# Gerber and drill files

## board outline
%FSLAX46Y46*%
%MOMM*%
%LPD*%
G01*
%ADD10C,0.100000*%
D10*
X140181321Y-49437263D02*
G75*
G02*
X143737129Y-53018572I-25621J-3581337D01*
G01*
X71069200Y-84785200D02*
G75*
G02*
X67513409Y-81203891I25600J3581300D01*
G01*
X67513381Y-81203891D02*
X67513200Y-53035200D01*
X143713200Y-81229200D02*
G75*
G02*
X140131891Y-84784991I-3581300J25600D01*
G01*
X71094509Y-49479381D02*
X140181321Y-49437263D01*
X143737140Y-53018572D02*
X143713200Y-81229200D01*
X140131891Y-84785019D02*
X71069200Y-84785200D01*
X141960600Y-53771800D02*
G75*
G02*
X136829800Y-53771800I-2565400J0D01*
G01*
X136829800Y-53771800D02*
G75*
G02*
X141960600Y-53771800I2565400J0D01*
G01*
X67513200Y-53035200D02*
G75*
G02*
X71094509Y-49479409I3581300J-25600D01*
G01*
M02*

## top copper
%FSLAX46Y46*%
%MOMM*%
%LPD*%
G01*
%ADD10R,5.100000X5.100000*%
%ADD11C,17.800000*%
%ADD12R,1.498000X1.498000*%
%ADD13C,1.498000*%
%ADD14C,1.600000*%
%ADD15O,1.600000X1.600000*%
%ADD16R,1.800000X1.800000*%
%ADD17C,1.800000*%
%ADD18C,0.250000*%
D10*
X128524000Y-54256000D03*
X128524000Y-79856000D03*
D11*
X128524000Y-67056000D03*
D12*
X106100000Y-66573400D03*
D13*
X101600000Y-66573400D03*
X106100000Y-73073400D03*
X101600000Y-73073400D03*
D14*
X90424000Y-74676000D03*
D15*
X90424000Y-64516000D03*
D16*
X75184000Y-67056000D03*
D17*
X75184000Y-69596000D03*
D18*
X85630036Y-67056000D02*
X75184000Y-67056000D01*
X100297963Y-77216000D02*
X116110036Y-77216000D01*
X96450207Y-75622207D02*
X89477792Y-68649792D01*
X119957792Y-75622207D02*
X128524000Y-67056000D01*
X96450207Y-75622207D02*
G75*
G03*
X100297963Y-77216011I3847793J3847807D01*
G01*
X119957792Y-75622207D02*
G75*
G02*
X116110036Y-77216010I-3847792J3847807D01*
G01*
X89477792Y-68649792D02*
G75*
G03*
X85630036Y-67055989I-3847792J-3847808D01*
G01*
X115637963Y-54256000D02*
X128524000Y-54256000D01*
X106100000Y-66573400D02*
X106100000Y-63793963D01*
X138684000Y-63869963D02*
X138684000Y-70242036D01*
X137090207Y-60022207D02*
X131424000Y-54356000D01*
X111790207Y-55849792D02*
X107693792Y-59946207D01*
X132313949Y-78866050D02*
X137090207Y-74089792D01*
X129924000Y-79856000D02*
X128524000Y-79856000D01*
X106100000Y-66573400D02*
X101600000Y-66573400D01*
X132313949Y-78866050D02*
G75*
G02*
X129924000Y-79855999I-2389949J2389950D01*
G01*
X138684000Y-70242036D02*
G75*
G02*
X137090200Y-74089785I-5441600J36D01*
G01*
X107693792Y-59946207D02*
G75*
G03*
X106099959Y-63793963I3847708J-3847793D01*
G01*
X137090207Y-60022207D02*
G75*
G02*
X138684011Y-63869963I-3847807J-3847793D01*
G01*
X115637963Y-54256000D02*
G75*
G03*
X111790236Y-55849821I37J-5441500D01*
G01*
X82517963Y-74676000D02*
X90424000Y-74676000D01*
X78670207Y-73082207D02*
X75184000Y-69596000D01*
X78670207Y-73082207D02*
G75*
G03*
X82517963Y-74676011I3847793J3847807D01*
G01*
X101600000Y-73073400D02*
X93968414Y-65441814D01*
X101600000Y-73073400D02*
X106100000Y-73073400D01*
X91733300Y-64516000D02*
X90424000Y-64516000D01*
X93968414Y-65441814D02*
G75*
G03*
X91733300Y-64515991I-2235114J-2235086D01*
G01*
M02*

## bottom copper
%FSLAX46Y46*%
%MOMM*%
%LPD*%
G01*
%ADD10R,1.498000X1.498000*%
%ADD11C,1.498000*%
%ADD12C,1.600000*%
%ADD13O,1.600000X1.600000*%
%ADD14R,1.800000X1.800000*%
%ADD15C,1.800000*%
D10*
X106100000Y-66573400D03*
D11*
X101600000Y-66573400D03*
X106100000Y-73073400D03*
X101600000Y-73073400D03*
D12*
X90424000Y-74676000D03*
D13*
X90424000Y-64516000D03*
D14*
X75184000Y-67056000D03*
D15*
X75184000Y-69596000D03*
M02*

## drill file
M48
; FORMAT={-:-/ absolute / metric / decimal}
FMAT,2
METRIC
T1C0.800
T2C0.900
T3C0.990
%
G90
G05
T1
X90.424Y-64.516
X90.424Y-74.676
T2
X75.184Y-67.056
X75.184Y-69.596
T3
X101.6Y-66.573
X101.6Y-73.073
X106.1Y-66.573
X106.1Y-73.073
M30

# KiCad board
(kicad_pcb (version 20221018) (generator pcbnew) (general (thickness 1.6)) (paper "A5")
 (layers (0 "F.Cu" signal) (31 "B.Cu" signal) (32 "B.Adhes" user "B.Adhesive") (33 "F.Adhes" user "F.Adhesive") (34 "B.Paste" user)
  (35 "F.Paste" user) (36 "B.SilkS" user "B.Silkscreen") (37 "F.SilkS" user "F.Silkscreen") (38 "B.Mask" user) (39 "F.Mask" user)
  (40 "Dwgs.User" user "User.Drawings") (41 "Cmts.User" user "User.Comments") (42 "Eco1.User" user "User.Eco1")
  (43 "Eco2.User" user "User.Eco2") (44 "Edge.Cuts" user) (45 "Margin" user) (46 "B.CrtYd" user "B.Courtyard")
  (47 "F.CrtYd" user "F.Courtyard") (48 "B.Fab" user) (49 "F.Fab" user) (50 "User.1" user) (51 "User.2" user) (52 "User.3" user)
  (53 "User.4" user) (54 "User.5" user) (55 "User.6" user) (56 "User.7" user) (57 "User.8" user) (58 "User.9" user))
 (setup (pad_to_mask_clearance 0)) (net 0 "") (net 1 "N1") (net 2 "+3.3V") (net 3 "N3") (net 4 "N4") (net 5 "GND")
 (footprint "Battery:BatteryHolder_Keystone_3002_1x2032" (layer "F.Cu") (at 128.524 67.056 -90)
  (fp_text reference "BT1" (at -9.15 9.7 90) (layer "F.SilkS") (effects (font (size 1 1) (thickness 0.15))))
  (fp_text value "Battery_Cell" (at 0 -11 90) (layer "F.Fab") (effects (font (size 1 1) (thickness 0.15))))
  (pad "1" smd rect (at -12.8 0 270) (size 5.1 5.1) (layers "F.Cu" "F.Paste" "F.Mask") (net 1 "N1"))
  (pad "1" smd rect (at 12.8 0 270) (size 5.1 5.1) (layers "F.Cu" "F.Paste" "F.Mask") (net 1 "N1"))
  (pad "2" smd circle (at 0 0 270) (size 17.8 17.8) (layers "F.Cu" "F.Mask") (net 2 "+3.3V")))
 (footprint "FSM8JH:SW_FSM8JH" (layer "F.Cu") (at 103.85 69.8234 -90)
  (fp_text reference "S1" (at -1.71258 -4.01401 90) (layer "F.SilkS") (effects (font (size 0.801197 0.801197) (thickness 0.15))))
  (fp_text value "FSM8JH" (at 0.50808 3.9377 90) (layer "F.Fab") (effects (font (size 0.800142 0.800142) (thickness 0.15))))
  (pad "1" thru_hole rect (at -3.25 -2.25 270) (size 1.498 1.498) (drill 0.99) (layers "*.Cu" "*.Mask") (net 1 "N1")
   (solder_mask_margin 0.102))
  (pad "2" thru_hole circle (at -3.25 2.25 270) (size 1.498 1.498) (drill 0.99) (layers "*.Cu" "*.Mask") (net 1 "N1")
   (solder_mask_margin 0.102))
  (pad "3" thru_hole circle (at 3.25 -2.25 270) (size 1.498 1.498) (drill 0.99) (layers "*.Cu" "*.Mask") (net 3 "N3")
   (solder_mask_margin 0.102))
  (pad "4" thru_hole circle (at 3.25 2.25 270) (size 1.498 1.498) (drill 0.99) (layers "*.Cu" "*.Mask") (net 3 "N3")
   (solder_mask_margin 0.102)))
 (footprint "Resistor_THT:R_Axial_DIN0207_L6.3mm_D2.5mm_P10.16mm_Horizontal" (layer "F.Cu") (at 90.424 74.676 90)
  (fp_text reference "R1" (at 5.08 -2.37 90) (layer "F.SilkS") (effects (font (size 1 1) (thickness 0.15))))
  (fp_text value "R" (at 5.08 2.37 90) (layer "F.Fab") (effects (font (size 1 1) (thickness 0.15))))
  (pad "1" thru_hole circle (at 0 0 90) (size 1.6 1.6) (drill 0.8) (layers "*.Cu" "*.Mask") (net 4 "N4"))
  (pad "2" thru_hole oval (at 10.16 0 90) (size 1.6 1.6) (drill 0.8) (layers "*.Cu" "*.Mask") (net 3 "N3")))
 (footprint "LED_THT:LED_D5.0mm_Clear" (layer "F.Cu") (at 75.184 67.056 -90)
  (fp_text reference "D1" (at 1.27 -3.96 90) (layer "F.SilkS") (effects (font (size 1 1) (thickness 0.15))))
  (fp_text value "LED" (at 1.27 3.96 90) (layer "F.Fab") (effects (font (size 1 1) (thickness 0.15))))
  (pad "1" thru_hole rect (at 0 0 270) (size 1.8 1.8) (drill 0.9) (layers "*.Cu" "*.Mask") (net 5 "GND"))
  (pad "2" thru_hole circle (at 2.54 0 270) (size 1.8 1.8) (drill 0.9) (layers "*.Cu" "*.Mask") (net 4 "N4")))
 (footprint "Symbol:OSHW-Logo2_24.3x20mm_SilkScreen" (layer "B.Cu") (at 128.27 71.12 180)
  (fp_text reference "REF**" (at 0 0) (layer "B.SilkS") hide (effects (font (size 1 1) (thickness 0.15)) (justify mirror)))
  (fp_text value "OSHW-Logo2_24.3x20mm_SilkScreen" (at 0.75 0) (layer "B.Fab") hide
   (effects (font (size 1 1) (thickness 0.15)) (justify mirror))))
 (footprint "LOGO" (layer "B.Cu") (at 86.868 58.42 180)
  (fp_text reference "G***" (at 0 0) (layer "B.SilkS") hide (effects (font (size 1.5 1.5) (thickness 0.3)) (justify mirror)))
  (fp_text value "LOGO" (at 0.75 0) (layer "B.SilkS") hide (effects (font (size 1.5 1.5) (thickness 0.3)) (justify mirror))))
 (gr_arc (start 140.181321 49.437263) (mid 142.6972 50.4952) (end 143.73714 53.018572) (stroke (width 0.1) (type default))
  (layer "Edge.Cuts"))
 (gr_arc (start 71.0692 84.7852) (mid 68.553321 83.727263) (end 67.513381 81.203891) (stroke (width 0.1) (type default)) (layer "Edge.Cuts"))
 (gr_line (start 67.513381 81.203891) (end 67.5132 53.0352) (stroke (width 0.1) (type default)) (layer "Edge.Cuts"))
 (gr_arc (start 143.7132 81.2292) (mid 142.655263 83.745079) (end 140.131891 84.785019) (stroke (width 0.1) (type default))
  (layer "Edge.Cuts"))
 (gr_line (start 71.094509 49.479381) (end 140.181321 49.437263) (stroke (width 0.1) (type default)) (layer "Edge.Cuts"))
 (gr_line (start 143.73714 53.018572) (end 143.7132 81.2292) (stroke (width 0.1) (type default)) (layer "Edge.Cuts"))
 (gr_line (start 140.131891 84.785019) (end 71.0692 84.7852) (stroke (width 0.1) (type default)) (layer "Edge.Cuts"))
 (gr_circle (center 139.3952 53.7718) (end 139.9032 56.2864) (stroke (width 0.1) (type default)) (fill none) (layer "Edge.Cuts"))
 (gr_arc (start 67.5132 53.0352) (mid 68.571137 50.519321) (end 71.094509 49.479381) (stroke (width 0.1) (type default)) (layer "Edge.Cuts"))
 (segment (start 85.630036 67.056) (end 75.184 67.056) (width 0.25) (layer "F.Cu") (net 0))
 (segment (start 100.297963 77.216) (end 116.110036 77.216) (width 0.25) (layer "F.Cu") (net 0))
 (segment (start 96.450207 75.622207) (end 89.477792 68.649792) (width 0.25) (layer "F.Cu") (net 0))
 (segment (start 119.957792 75.622207) (end 128.524 67.056) (width 0.25) (layer "F.Cu") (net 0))
 (arc (start 96.450207 75.622207) (mid 98.215572 76.801786) (end 100.297963 77.216) (width 0.25) (layer "F.Cu") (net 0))
 (arc (start 119.957792 75.622207) (mid 118.192426 76.801786) (end 116.110036 77.216) (width 0.25) (layer "F.Cu") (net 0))
 (arc (start 89.477792 68.649792) (mid 87.712426 67.470213) (end 85.630036 67.056) (width 0.25) (layer "F.Cu") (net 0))
 (segment (start 115.637963 54.256) (end 128.524 54.256) (width 0.25) (layer "F.Cu") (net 1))
 (segment (start 106.1 66.5734) (end 106.1 63.793963) (width 0.25) (layer "F.Cu") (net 1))
 (segment (start 138.684 63.869963) (end 138.684 70.242036) (width 0.25) (layer "F.Cu") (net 1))
 (segment (start 137.090207 60.022207) (end 131.424 54.356) (width 0.25) (layer "F.Cu") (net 1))
 (segment (start 111.790207 55.849792) (end 107.693792 59.946207) (width 0.25) (layer "F.Cu") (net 1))
 (segment (start 132.313949 78.86605) (end 137.090207 74.089792) (width 0.25) (layer "F.Cu") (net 1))
 (segment (start 129.924 79.856) (end 128.524 79.856) (width 0.25) (layer "F.Cu") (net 1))
 (segment (start 106.1 66.5734) (end 101.6 66.5734) (width 0.25) (layer "F.Cu") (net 1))
 (arc (start 132.313949 78.86605) (mid 131.217431 79.59872) (end 129.924 79.856) (width 0.25) (layer "F.Cu") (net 1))
 (arc (start 138.684 70.242036) (mid 138.269786 72.324426) (end 137.090207 74.089792) (width 0.25) (layer "F.Cu") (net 1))
 (arc (start 107.693792 59.946207) (mid 106.514213 61.711572) (end 106.1 63.793963) (width 0.25) (layer "F.Cu") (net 1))
 (arc (start 137.090207 60.022207) (mid 138.269786 61.787572) (end 138.684 63.869963) (width 0.25) (layer "F.Cu") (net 1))
 (arc (start 115.637963 54.256) (mid 113.555572 54.670213) (end 111.790207 55.849792) (width 0.25) (layer "F.Cu") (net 1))
 (segment (start 82.517963 74.676) (end 90.424 74.676) (width 0.25) (layer "F.Cu") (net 4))
 (segment (start 78.670207 73.082207) (end 75.184 69.596) (width 0.25) (layer "F.Cu") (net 4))
 (arc (start 78.670207 73.082207) (mid 80.435572 74.261786) (end 82.517963 74.676) (width 0.25) (layer "F.Cu") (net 4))
 (segment (start 101.6 73.0734) (end 93.968414 65.441814) (width 0.25) (layer "F.Cu") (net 3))
 (segment (start 101.6 73.0734) (end 106.1 73.0734) (width 0.25) (layer "F.Cu") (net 3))
 (segment (start 91.7333 64.516) (end 90.424 64.516) (width 0.25) (layer "F.Cu") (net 3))
 (arc (start 93.968414 65.441814) (mid 92.942935 64.756611) (end 91.7333 64.516) (width 0.25) (layer "F.Cu") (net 3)))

